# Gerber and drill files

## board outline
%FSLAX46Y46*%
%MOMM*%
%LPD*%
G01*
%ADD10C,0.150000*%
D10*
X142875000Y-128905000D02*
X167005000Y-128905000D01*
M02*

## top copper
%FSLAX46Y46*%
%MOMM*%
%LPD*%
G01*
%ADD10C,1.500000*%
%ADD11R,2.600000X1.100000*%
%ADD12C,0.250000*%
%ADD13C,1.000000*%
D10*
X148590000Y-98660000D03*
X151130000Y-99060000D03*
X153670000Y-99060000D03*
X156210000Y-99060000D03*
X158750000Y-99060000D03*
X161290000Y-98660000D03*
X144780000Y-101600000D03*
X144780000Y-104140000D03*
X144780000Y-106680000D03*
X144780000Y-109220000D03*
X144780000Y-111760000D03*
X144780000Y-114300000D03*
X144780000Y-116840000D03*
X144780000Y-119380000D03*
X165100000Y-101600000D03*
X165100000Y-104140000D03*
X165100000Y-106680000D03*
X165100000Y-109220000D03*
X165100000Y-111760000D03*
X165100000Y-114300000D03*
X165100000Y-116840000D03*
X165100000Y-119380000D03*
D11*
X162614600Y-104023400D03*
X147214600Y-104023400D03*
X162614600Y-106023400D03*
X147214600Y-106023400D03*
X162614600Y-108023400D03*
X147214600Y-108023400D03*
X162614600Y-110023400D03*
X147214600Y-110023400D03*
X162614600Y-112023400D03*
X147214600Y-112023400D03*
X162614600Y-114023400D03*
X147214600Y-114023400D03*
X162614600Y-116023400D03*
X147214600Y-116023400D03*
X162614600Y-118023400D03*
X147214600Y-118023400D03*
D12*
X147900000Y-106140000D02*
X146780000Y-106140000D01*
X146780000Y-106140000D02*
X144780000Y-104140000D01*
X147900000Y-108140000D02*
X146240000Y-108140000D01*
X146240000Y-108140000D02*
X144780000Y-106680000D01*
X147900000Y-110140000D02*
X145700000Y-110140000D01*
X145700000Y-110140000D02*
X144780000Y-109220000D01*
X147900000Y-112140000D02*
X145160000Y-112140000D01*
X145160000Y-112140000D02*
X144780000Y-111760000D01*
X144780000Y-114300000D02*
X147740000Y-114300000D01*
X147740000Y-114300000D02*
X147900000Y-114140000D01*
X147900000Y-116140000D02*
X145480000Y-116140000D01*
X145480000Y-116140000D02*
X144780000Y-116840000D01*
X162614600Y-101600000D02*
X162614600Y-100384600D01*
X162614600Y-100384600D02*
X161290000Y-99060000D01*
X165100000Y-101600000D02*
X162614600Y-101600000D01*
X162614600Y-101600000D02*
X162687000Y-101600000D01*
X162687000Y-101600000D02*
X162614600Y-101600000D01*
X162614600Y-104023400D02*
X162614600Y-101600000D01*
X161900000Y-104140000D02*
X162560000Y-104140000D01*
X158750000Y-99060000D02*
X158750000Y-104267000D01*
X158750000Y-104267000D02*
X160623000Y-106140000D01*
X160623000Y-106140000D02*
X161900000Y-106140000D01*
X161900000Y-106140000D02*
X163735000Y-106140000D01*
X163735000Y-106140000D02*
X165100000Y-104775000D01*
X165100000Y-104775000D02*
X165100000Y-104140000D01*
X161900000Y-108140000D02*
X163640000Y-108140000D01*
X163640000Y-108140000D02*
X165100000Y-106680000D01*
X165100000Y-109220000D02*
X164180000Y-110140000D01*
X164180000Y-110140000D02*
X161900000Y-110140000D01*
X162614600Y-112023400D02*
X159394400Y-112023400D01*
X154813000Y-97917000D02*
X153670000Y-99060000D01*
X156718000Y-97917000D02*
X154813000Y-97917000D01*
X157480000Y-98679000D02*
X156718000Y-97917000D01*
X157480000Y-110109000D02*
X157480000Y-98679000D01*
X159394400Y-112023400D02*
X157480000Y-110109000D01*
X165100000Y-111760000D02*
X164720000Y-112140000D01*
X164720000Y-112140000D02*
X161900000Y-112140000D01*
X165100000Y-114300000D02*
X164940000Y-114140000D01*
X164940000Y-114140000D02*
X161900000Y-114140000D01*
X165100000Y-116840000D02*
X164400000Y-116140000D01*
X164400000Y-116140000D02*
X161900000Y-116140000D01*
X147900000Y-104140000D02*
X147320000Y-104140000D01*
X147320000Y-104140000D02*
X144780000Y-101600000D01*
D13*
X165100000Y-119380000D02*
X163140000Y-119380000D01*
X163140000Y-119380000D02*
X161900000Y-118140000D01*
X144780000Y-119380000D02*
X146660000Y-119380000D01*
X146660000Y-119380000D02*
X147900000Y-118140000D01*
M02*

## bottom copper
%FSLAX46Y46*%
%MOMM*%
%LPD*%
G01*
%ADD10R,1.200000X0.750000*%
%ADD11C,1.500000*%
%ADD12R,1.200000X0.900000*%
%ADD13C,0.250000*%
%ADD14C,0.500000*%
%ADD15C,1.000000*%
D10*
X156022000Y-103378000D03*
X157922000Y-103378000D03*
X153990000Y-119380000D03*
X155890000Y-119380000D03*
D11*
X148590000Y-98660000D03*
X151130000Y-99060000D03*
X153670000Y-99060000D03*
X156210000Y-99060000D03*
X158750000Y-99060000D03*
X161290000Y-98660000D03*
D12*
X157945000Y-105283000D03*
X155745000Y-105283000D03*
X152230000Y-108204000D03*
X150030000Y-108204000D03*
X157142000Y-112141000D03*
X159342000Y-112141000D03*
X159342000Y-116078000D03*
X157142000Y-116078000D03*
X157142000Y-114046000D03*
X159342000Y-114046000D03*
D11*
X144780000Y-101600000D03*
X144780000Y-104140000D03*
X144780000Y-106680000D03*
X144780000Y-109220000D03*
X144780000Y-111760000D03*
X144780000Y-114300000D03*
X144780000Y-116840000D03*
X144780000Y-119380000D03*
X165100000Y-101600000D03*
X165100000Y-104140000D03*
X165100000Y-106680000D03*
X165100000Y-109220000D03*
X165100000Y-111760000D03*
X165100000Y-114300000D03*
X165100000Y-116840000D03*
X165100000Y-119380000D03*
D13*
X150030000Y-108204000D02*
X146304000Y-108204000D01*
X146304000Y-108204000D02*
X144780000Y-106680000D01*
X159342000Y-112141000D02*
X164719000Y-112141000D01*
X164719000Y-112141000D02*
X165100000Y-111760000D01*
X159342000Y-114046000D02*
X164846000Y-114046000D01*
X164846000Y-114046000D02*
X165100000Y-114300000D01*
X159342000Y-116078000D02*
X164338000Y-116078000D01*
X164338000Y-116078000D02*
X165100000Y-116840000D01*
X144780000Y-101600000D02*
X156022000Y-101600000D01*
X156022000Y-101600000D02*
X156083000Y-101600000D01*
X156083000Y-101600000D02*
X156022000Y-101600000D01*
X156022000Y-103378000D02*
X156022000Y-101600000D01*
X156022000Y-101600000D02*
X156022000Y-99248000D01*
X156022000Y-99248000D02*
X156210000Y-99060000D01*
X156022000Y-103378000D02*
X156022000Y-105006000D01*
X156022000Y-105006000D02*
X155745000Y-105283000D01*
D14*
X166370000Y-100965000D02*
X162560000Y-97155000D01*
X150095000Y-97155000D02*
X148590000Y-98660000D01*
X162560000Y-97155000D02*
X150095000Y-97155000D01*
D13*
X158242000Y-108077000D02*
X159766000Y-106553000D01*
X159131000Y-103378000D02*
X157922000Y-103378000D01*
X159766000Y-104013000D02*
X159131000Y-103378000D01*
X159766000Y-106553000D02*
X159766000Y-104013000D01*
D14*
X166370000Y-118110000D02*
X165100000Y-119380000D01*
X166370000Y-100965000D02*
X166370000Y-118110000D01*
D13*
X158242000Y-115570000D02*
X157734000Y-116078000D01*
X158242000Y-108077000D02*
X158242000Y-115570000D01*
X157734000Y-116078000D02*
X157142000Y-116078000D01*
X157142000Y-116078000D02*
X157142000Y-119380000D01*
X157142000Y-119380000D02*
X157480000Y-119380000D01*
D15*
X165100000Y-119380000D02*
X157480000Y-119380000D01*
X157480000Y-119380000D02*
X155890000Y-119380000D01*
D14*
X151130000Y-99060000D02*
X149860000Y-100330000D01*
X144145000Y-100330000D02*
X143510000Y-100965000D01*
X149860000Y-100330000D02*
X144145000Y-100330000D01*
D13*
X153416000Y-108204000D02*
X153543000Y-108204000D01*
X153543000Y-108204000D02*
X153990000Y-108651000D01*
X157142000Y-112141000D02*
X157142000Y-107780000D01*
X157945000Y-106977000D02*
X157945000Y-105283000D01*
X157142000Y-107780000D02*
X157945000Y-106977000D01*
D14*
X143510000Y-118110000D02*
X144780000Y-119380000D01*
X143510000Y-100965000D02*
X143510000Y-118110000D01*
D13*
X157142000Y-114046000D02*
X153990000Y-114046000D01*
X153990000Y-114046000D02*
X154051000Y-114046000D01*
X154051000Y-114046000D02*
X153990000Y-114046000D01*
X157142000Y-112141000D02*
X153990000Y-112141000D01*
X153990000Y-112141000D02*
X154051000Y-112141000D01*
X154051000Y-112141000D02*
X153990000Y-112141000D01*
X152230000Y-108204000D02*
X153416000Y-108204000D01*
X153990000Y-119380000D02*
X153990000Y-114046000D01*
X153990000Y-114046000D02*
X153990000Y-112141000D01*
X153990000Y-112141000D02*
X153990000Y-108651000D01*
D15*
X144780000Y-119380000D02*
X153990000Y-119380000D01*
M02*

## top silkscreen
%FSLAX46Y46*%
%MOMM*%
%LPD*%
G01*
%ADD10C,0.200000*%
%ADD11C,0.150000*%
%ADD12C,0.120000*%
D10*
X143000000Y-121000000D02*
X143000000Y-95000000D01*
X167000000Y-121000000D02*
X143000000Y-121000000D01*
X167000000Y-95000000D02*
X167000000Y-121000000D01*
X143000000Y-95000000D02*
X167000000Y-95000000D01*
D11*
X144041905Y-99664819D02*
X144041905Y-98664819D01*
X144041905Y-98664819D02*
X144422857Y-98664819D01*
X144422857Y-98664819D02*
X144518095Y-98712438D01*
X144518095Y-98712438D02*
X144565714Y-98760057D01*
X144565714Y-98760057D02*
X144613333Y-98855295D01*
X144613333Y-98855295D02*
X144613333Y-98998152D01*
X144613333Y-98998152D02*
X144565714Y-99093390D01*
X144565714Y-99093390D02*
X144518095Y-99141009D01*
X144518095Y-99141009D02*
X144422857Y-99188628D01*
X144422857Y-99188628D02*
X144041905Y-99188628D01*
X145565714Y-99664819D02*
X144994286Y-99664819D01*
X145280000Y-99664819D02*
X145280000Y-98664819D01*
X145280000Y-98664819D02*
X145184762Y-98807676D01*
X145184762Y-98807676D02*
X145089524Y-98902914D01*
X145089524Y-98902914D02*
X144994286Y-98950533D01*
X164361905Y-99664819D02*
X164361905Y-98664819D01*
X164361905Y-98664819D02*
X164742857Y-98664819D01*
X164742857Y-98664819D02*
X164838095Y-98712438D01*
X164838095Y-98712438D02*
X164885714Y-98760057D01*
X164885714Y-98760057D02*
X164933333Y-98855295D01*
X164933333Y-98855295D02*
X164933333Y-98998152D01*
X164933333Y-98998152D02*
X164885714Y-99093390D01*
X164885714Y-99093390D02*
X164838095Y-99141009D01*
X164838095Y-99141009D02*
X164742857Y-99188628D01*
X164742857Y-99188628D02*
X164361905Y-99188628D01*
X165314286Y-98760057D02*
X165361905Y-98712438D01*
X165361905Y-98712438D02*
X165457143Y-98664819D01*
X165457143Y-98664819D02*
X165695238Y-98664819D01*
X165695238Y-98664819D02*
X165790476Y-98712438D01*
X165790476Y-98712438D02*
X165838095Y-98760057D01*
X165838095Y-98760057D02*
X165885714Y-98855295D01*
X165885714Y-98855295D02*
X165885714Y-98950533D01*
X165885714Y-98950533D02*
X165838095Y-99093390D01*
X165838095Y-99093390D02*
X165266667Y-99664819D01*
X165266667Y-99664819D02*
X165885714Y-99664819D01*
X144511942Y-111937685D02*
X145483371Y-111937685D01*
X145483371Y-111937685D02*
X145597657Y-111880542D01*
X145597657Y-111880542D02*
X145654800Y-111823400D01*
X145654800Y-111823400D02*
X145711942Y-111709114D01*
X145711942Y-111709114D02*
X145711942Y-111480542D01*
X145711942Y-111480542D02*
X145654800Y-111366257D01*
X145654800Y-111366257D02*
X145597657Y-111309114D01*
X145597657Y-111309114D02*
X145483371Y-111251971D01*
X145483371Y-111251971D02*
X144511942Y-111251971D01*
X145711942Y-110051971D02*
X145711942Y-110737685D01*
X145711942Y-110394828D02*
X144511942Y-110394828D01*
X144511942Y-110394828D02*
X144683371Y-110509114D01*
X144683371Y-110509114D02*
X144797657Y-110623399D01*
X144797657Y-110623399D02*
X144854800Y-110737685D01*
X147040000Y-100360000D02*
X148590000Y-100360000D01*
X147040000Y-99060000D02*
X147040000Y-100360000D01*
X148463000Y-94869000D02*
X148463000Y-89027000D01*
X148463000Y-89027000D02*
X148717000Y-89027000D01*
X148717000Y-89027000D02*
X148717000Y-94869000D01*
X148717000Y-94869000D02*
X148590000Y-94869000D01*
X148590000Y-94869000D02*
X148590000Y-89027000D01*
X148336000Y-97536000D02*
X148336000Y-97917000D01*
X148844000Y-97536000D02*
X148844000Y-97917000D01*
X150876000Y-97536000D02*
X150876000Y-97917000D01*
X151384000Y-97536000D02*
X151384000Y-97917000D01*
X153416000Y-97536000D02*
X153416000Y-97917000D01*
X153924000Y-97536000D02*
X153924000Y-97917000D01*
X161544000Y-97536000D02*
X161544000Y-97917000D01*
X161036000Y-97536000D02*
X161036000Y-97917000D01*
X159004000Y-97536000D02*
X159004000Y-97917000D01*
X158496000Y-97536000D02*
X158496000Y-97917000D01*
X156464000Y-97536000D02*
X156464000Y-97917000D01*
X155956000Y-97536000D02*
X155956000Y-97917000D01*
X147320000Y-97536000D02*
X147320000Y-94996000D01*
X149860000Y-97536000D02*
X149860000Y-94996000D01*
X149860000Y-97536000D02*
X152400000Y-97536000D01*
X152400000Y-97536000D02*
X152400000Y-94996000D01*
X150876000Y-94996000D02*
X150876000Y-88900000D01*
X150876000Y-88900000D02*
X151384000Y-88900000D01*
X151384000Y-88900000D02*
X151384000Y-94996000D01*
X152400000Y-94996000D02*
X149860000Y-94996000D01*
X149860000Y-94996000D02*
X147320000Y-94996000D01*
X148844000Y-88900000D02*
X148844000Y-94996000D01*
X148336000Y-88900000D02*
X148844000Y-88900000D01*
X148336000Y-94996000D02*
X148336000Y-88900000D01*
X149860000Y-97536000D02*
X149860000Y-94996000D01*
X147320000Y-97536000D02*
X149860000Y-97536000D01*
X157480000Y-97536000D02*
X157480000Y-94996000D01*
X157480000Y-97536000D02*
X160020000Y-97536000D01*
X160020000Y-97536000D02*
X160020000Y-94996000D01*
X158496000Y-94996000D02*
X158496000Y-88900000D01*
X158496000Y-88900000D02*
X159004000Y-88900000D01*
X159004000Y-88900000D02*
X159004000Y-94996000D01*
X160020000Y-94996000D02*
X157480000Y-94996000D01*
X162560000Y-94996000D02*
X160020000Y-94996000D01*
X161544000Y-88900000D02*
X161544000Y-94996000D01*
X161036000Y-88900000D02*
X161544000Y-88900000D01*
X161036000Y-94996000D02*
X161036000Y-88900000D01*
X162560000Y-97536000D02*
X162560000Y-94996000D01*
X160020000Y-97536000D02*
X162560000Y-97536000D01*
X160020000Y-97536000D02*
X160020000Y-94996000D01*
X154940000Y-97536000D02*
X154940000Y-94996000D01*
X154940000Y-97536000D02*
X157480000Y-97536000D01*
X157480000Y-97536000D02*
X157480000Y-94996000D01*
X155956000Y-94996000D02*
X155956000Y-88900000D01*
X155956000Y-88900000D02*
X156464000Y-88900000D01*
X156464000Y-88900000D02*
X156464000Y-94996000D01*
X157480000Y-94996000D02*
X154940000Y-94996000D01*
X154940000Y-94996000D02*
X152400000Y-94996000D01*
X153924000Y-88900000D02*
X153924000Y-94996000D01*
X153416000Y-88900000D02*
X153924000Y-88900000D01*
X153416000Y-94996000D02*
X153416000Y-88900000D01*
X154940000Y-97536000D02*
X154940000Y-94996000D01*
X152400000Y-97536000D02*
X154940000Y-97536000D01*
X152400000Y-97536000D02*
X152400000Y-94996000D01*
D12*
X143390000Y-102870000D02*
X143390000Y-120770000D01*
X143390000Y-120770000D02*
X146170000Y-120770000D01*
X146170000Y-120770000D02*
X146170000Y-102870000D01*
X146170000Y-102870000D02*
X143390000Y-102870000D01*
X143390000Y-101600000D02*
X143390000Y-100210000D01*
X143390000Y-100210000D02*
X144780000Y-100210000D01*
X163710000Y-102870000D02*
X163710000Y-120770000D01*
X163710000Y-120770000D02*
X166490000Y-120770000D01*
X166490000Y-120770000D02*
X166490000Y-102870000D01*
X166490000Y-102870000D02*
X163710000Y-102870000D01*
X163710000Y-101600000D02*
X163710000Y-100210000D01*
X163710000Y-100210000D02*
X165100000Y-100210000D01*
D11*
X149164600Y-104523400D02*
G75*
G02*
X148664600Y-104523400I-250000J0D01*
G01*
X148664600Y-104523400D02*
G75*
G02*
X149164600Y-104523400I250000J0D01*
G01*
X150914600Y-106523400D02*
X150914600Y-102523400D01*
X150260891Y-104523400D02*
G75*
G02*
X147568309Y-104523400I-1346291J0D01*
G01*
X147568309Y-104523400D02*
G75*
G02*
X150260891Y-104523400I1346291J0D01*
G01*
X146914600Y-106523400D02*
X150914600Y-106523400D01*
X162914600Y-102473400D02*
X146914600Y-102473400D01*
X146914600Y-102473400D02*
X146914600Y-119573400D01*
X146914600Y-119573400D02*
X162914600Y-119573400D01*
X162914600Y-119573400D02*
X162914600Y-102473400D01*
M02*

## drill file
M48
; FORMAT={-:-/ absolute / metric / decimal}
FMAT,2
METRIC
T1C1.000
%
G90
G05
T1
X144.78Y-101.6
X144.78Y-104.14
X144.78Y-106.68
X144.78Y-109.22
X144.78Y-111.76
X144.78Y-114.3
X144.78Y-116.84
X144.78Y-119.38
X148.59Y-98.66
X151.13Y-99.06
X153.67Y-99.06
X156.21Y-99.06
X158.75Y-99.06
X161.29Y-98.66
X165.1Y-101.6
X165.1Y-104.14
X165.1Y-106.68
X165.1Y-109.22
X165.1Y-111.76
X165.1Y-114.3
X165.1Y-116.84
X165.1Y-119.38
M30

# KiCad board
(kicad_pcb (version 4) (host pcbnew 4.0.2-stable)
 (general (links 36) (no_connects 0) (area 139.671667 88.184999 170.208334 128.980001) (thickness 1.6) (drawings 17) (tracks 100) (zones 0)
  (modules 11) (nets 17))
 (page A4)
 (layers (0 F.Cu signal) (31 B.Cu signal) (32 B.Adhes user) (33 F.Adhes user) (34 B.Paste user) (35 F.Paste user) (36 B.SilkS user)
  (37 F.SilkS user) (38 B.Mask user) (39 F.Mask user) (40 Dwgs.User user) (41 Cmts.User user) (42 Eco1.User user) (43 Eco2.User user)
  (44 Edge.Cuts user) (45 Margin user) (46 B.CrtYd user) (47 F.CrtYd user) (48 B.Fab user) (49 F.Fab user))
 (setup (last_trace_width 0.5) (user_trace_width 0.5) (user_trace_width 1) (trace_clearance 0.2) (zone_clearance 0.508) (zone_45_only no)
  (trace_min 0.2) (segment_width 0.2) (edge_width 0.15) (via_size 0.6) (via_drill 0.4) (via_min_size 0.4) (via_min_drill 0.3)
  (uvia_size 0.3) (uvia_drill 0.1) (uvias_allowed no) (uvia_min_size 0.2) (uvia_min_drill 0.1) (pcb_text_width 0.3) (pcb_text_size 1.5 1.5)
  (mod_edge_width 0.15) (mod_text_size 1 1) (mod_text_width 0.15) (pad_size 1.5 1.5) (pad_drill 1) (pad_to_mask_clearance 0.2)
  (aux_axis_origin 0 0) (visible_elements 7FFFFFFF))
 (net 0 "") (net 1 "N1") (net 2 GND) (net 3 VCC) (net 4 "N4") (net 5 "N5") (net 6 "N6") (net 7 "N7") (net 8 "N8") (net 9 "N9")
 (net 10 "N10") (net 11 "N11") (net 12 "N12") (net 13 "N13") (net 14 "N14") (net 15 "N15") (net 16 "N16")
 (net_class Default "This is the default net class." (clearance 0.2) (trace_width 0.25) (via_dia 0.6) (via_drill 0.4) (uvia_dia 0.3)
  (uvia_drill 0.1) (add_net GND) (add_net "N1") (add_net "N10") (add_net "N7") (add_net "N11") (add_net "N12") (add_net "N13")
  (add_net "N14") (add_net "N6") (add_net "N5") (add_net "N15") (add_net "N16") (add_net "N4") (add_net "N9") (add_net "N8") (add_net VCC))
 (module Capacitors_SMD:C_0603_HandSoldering (layer B.Cu) (at 156.972 103.378)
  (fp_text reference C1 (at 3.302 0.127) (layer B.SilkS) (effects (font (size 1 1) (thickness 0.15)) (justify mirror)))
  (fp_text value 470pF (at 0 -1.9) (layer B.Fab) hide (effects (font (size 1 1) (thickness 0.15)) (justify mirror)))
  (pad 1 smd rect (at -0.95 0) (size 1.2 0.75) (layers B.Cu B.Paste B.Mask) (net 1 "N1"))
  (pad 2 smd rect (at 0.95 0) (size 1.2 0.75) (layers B.Cu B.Paste B.Mask) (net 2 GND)))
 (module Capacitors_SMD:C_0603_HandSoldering (layer B.Cu) (at 154.94 119.38)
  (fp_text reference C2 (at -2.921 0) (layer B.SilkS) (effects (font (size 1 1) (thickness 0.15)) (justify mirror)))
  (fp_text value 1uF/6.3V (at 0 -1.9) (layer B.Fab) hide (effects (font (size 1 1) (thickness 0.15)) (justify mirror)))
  (pad 1 smd rect (at -0.95 0) (size 1.2 0.75) (layers B.Cu B.Paste B.Mask) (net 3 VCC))
  (pad 2 smd rect (at 0.95 0) (size 1.2 0.75) (layers B.Cu B.Paste B.Mask) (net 2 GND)))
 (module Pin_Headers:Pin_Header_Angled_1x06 (layer F.Cu) (at 148.59 99.06 90)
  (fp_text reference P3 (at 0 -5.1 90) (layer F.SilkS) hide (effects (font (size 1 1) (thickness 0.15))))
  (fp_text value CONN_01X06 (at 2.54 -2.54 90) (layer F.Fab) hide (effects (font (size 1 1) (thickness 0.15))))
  (fp_line (start -1.3 -1.55) (end -1.3 0) (layer F.SilkS) (width 0.15))
  (fp_line (start 0 -1.55) (end -1.3 -1.55) (layer F.SilkS) (width 0.15))
  (fp_line (start 4.191 -0.127) (end 10.033 -0.127) (layer F.SilkS) (width 0.15))
  (fp_line (start 10.033 -0.127) (end 10.033 0.127) (layer F.SilkS) (width 0.15))
  (fp_line (start 10.033 0.127) (end 4.191 0.127) (layer F.SilkS) (width 0.15))
  (fp_line (start 4.191 0.127) (end 4.191 0) (layer F.SilkS) (width 0.15))
  (fp_line (start 4.191 0) (end 10.033 0) (layer F.SilkS) (width 0.15))
  (fp_line (start 1.524 -0.254) (end 1.143 -0.254) (layer F.SilkS) (width 0.15))
  (fp_line (start 1.524 0.254) (end 1.143 0.254) (layer F.SilkS) (width 0.15))
  (fp_line (start 1.524 2.286) (end 1.143 2.286) (layer F.SilkS) (width 0.15))
  (fp_line (start 1.524 2.794) (end 1.143 2.794) (layer F.SilkS) (width 0.15))
  (fp_line (start 1.524 4.826) (end 1.143 4.826) (layer F.SilkS) (width 0.15))
  (fp_line (start 1.524 5.334) (end 1.143 5.334) (layer F.SilkS) (width 0.15))
  (fp_line (start 1.524 12.954) (end 1.143 12.954) (layer F.SilkS) (width 0.15))
  (fp_line (start 1.524 12.446) (end 1.143 12.446) (layer F.SilkS) (width 0.15))
  (fp_line (start 1.524 10.414) (end 1.143 10.414) (layer F.SilkS) (width 0.15))
  (fp_line (start 1.524 9.906) (end 1.143 9.906) (layer F.SilkS) (width 0.15))
  (fp_line (start 1.524 7.874) (end 1.143 7.874) (layer F.SilkS) (width 0.15))
  (fp_line (start 1.524 7.366) (end 1.143 7.366) (layer F.SilkS) (width 0.15))
  (fp_line (start 1.524 -1.27) (end 4.064 -1.27) (layer F.SilkS) (width 0.15))
  (fp_line (start 1.524 1.27) (end 4.064 1.27) (layer F.SilkS) (width 0.15))
  (fp_line (start 1.524 1.27) (end 1.524 3.81) (layer F.SilkS) (width 0.15))
  (fp_line (start 1.524 3.81) (end 4.064 3.81) (layer F.SilkS) (width 0.15))
  (fp_line (start 4.064 2.286) (end 10.16 2.286) (layer F.SilkS) (width 0.15))
  (fp_line (start 10.16 2.286) (end 10.16 2.794) (layer F.SilkS) (width 0.15))
  (fp_line (start 10.16 2.794) (end 4.064 2.794) (layer F.SilkS) (width 0.15))
  (fp_line (start 4.064 3.81) (end 4.064 1.27) (layer F.SilkS) (width 0.15))
  (fp_line (start 4.064 1.27) (end 4.064 -1.27) (layer F.SilkS) (width 0.15))
  (fp_line (start 10.16 0.254) (end 4.064 0.254) (layer F.SilkS) (width 0.15))
  (fp_line (start 10.16 -0.254) (end 10.16 0.254) (layer F.SilkS) (width 0.15))
  (fp_line (start 4.064 -0.254) (end 10.16 -0.254) (layer F.SilkS) (width 0.15))
  (fp_line (start 1.524 1.27) (end 4.064 1.27) (layer F.SilkS) (width 0.15))
  (fp_line (start 1.524 -1.27) (end 1.524 1.27) (layer F.SilkS) (width 0.15))
  (fp_line (start 1.524 8.89) (end 4.064 8.89) (layer F.SilkS) (width 0.15))
  (fp_line (start 1.524 8.89) (end 1.524 11.43) (layer F.SilkS) (width 0.15))
  (fp_line (start 1.524 11.43) (end 4.064 11.43) (layer F.SilkS) (width 0.15))
  (fp_line (start 4.064 9.906) (end 10.16 9.906) (layer F.SilkS) (width 0.15))
  (fp_line (start 10.16 9.906) (end 10.16 10.414) (layer F.SilkS) (width 0.15))
  (fp_line (start 10.16 10.414) (end 4.064 10.414) (layer F.SilkS) (width 0.15))
  (fp_line (start 4.064 11.43) (end 4.064 8.89) (layer F.SilkS) (width 0.15))
  (fp_line (start 4.064 13.97) (end 4.064 11.43) (layer F.SilkS) (width 0.15))
  (fp_line (start 10.16 12.954) (end 4.064 12.954) (layer F.SilkS) (width 0.15))
  (fp_line (start 10.16 12.446) (end 10.16 12.954) (layer F.SilkS) (width 0.15))
  (fp_line (start 4.064 12.446) (end 10.16 12.446) (layer F.SilkS) (width 0.15))
  (fp_line (start 1.524 13.97) (end 4.064 13.97) (layer F.SilkS) (width 0.15))
  (fp_line (start 1.524 11.43) (end 1.524 13.97) (layer F.SilkS) (width 0.15))
  (fp_line (start 1.524 11.43) (end 4.064 11.43) (layer F.SilkS) (width 0.15))
  (fp_line (start 1.524 6.35) (end 4.064 6.35) (layer F.SilkS) (width 0.15))
  (fp_line (start 1.524 6.35) (end 1.524 8.89) (layer F.SilkS) (width 0.15))
  (fp_line (start 1.524 8.89) (end 4.064 8.89) (layer F.SilkS) (width 0.15))
  (fp_line (start 4.064 7.366) (end 10.16 7.366) (layer F.SilkS) (width 0.15))
  (fp_line (start 10.16 7.366) (end 10.16 7.874) (layer F.SilkS) (width 0.15))
  (fp_line (start 10.16 7.874) (end 4.064 7.874) (layer F.SilkS) (width 0.15))
  (fp_line (start 4.064 8.89) (end 4.064 6.35) (layer F.SilkS) (width 0.15))
  (fp_line (start 4.064 6.35) (end 4.064 3.81) (layer F.SilkS) (width 0.15))
  (fp_line (start 10.16 5.334) (end 4.064 5.334) (layer F.SilkS) (width 0.15))
  (fp_line (start 10.16 4.826) (end 10.16 5.334) (layer F.SilkS) (width 0.15))
  (fp_line (start 4.064 4.826) (end 10.16 4.826) (layer F.SilkS) (width 0.15))
  (fp_line (start 1.524 6.35) (end 4.064 6.35) (layer F.SilkS) (width 0.15))
  (fp_line (start 1.524 3.81) (end 1.524 6.35) (layer F.SilkS) (width 0.15))
  (fp_line (start 1.524 3.81) (end 4.064 3.81) (layer F.SilkS) (width 0.15))
  (pad 1 thru_hole circle (at 0.4 0 90) (size 1.5 1.5) (drill 1) (layers *.Cu *.Mask) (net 2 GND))
  (pad 2 thru_hole circle (at 0 2.54 90) (size 1.5 1.5) (drill 1) (layers *.Cu *.Mask) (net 3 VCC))
  (pad 3 thru_hole circle (at 0 5.08 90) (size 1.5 1.5) (drill 1) (layers *.Cu *.Mask) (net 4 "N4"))
  (pad 4 thru_hole circle (at 0 7.62 90) (size 1.5 1.5) (drill 1) (layers *.Cu *.Mask) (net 1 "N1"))
  (pad 5 thru_hole circle (at 0 10.16 90) (size 1.5 1.5) (drill 1) (layers *.Cu *.Mask) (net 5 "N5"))
  (pad 6 thru_hole circle (at 0.4 12.7 90) (size 1.5 1.5) (drill 1) (layers *.Cu *.Mask) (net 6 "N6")))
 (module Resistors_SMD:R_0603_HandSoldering (layer B.Cu) (at 156.845 105.283 180)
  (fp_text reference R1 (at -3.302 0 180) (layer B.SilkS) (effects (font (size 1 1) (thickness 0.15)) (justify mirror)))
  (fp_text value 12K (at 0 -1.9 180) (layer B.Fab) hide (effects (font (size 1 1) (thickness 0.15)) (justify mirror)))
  (pad 1 smd rect (at -1.1 0 180) (size 1.2 0.9) (layers B.Cu B.Paste B.Mask) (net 3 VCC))
  (pad 2 smd rect (at 1.1 0 180) (size 1.2 0.9) (layers B.Cu B.Paste B.Mask) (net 1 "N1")))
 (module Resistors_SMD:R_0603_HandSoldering (layer B.Cu) (at 151.13 108.204 180)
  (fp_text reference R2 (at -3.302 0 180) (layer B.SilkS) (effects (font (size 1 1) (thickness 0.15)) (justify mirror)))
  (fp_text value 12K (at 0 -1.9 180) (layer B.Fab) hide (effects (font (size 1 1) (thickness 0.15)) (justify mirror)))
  (pad 1 smd rect (at -1.1 0 180) (size 1.2 0.9) (layers B.Cu B.Paste B.Mask) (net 3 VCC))
  (pad 2 smd rect (at 1.1 0 180) (size 1.2 0.9) (layers B.Cu B.Paste B.Mask) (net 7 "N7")))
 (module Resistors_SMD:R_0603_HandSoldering (layer B.Cu) (at 158.242 112.141)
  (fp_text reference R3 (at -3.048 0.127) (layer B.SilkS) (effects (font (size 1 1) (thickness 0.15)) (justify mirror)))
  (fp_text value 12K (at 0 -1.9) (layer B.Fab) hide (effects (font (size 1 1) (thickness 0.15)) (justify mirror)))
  (pad 1 smd rect (at -1.1 0) (size 1.2 0.9) (layers B.Cu B.Paste B.Mask) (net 3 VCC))
  (pad 2 smd rect (at 1.1 0) (size 1.2 0.9) (layers B.Cu B.Paste B.Mask) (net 4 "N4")))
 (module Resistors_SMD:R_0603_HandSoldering (layer B.Cu) (at 158.242 116.078 180)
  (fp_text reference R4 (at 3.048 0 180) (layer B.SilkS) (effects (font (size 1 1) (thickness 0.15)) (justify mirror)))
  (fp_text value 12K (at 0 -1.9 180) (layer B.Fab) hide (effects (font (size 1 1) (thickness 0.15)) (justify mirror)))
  (pad 1 smd rect (at -1.1 0 180) (size 1.2 0.9) (layers B.Cu B.Paste B.Mask) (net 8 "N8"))
  (pad 2 smd rect (at 1.1 0 180) (size 1.2 0.9) (layers B.Cu B.Paste B.Mask) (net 2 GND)))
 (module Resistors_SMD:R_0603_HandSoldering (layer B.Cu) (at 158.242 114.046)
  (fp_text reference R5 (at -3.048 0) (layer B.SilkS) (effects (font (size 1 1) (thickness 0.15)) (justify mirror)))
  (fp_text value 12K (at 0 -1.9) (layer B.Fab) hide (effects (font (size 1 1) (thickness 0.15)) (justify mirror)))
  (pad 1 smd rect (at -1.1 0) (size 1.2 0.9) (layers B.Cu B.Paste B.Mask) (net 3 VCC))
  (pad 2 smd rect (at 1.1 0) (size 1.2 0.9) (layers B.Cu B.Paste B.Mask) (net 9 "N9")))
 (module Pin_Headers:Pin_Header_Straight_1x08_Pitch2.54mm (layer F.Cu) (at 144.78 101.6)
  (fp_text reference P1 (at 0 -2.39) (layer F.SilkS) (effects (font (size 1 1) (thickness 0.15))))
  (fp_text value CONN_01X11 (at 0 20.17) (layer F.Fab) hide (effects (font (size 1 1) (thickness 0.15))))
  (fp_line (start -1.39 1.27) (end -1.39 19.17) (layer F.SilkS) (width 0.12))
  (fp_line (start -1.39 19.17) (end 1.39 19.17) (layer F.SilkS) (width 0.12))
  (fp_line (start 1.39 19.17) (end 1.39 1.27) (layer F.SilkS) (width 0.12))
  (fp_line (start 1.39 1.27) (end -1.39 1.27) (layer F.SilkS) (width 0.12))
  (fp_line (start -1.39 0) (end -1.39 -1.39) (layer F.SilkS) (width 0.12))
  (fp_line (start -1.39 -1.39) (end 0 -1.39) (layer F.SilkS) (width 0.12))
  (pad 1 thru_hole circle (at 0 0) (size 1.5 1.5) (drill 1) (layers *.Cu *.Mask) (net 1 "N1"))
  (pad 2 thru_hole circle (at 0 2.54) (size 1.5 1.5) (drill 1) (layers *.Cu *.Mask) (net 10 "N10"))
  (pad 3 thru_hole circle (at 0 5.08) (size 1.5 1.5) (drill 1) (layers *.Cu *.Mask) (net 7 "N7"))
  (pad 4 thru_hole circle (at 0 7.62) (size 1.5 1.5) (drill 1) (layers *.Cu *.Mask) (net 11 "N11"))
  (pad 5 thru_hole circle (at 0 10.16) (size 1.5 1.5) (drill 1) (layers *.Cu *.Mask) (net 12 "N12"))
  (pad 6 thru_hole circle (at 0 12.7) (size 1.5 1.5) (drill 1) (layers *.Cu *.Mask) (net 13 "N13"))
  (pad 7 thru_hole circle (at 0 15.24) (size 1.5 1.5) (drill 1) (layers *.Cu *.Mask) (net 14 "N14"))
  (pad 8 thru_hole circle (at 0 17.78) (size 1.5 1.5) (drill 1) (layers *.Cu *.Mask) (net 3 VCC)))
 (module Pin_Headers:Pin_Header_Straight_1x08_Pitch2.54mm (layer F.Cu) (at 165.1 101.6)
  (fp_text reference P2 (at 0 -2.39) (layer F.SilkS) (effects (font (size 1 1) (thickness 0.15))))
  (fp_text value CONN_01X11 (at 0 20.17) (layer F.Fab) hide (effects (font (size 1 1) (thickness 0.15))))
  (fp_line (start -1.39 1.27) (end -1.39 19.17) (layer F.SilkS) (width 0.12))
  (fp_line (start -1.39 19.17) (end 1.39 19.17) (layer F.SilkS) (width 0.12))
  (fp_line (start 1.39 19.17) (end 1.39 1.27) (layer F.SilkS) (width 0.12))
  (fp_line (start 1.39 1.27) (end -1.39 1.27) (layer F.SilkS) (width 0.12))
  (fp_line (start -1.39 0) (end -1.39 -1.39) (layer F.SilkS) (width 0.12))
  (fp_line (start -1.39 -1.39) (end 0 -1.39) (layer F.SilkS) (width 0.12))
  (pad 1 thru_hole circle (at 0 0) (size 1.5 1.5) (drill 1) (layers *.Cu *.Mask) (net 6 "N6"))
  (pad 2 thru_hole circle (at 0 2.54) (size 1.5 1.5) (drill 1) (layers *.Cu *.Mask) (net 5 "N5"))
  (pad 3 thru_hole circle (at 0 5.08) (size 1.5 1.5) (drill 1) (layers *.Cu *.Mask) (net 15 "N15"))
  (pad 4 thru_hole circle (at 0 7.62) (size 1.5 1.5) (drill 1) (layers *.Cu *.Mask) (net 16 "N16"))
  (pad 5 thru_hole circle (at 0 10.16) (size 1.5 1.5) (drill 1) (layers *.Cu *.Mask) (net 4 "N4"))
  (pad 6 thru_hole circle (at 0 12.7) (size 1.5 1.5) (drill 1) (layers *.Cu *.Mask) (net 9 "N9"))
  (pad 7 thru_hole circle (at 0 15.24) (size 1.5 1.5) (drill 1) (layers *.Cu *.Mask) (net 8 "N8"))
  (pad 8 thru_hole circle (at 0 17.78) (size 1.5 1.5) (drill 1) (layers *.Cu *.Mask) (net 2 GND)))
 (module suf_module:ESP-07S (layer F.Cu) (at 154.9146 111.0234)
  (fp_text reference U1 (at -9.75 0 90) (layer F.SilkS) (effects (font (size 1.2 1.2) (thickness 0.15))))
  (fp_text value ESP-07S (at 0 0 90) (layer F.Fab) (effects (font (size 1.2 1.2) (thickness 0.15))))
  (fp_circle (center -6 -6.5) (end -6 -6.75) (layer F.SilkS) (width 0.15))
  (fp_line (start -4 -4.5) (end -4 -8.5) (layer F.SilkS) (width 0.15))
  (fp_circle (center -6 -6.5) (end -5.5 -7.75) (layer F.SilkS) (width 0.15))
  (fp_line (start -8 -4.5) (end -4 -4.5) (layer F.SilkS) (width 0.15))
  (fp_line (start 8 -8.55) (end -8 -8.55) (layer F.SilkS) (width 0.15))
  (fp_line (start -8 -8.55) (end -8 8.55) (layer F.SilkS) (width 0.15))
  (fp_line (start -8 8.55) (end 8 8.55) (layer F.SilkS) (width 0.15))
  (fp_line (start 8 8.55) (end 8 -8.55) (layer F.SilkS) (width 0.15))
  (pad 16 smd rect (at 7.7 -7 270) (size 1.1 2.6) (layers F.Cu F.Paste F.Mask) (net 6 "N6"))
  (pad 1 smd rect (at -7.7 -7 270) (size 1.1 2.6) (layers F.Cu F.Paste F.Mask) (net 1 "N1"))
  (pad 15 smd rect (at 7.7 -5 270) (size 1.1 2.6) (layers F.Cu F.Paste F.Mask) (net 5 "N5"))
  (pad 2 smd rect (at -7.7 -5 270) (size 1.1 2.6) (layers F.Cu F.Paste F.Mask) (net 10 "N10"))
  (pad 14 smd rect (at 7.7 -3 270) (size 1.1 2.6) (layers F.Cu F.Paste F.Mask) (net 15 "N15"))
  (pad 3 smd rect (at -7.7 -3 270) (size 1.1 2.6) (layers F.Cu F.Paste F.Mask) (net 7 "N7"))
  (pad 13 smd rect (at 7.7 -1 270) (size 1.1 2.6) (layers F.Cu F.Paste F.Mask) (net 16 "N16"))
  (pad 4 smd rect (at -7.7 -1 270) (size 1.1 2.6) (layers F.Cu F.Paste F.Mask) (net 11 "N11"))
  (pad 12 smd rect (at 7.7 1 270) (size 1.1 2.6) (layers F.Cu F.Paste F.Mask) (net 4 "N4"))
  (pad 5 smd rect (at -7.7 1 270) (size 1.1 2.6) (layers F.Cu F.Paste F.Mask) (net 12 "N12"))
  (pad 11 smd rect (at 7.7 3 270) (size 1.1 2.6) (layers F.Cu F.Paste F.Mask) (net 9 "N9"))
  (pad 6 smd rect (at -7.7 3 270) (size 1.1 2.6) (layers F.Cu F.Paste F.Mask) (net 13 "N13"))
  (pad 10 smd rect (at 7.7 5 270) (size 1.1 2.6) (layers F.Cu F.Paste F.Mask) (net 8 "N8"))
  (pad 7 smd rect (at -7.7 5 270) (size 1.1 2.6) (layers F.Cu F.Paste F.Mask) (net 14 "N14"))
  (pad 9 smd rect (at 7.7 7 270) (size 1.1 2.6) (layers F.Cu F.Paste F.Mask) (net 2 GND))
  (pad 8 smd rect (at -7.7 7 270) (size 1.1 2.6) (layers F.Cu F.Paste F.Mask) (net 3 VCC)))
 (gr_line (start 143 121) (end 143 95) (angle 90) (layer F.SilkS) (width 0.2))
 (gr_line (start 167 121) (end 143 121) (angle 90) (layer F.SilkS) (width 0.2))
 (gr_line (start 167 95) (end 167 121) (angle 90) (layer F.SilkS) (width 0.2))
 (gr_line (start 143 95) (end 167 95) (angle 90) (layer F.SilkS) (width 0.2))
 (gr_line (start 142.875 128.905) (end 167.005 128.905) (angle 90) (layer Edge.Cuts) (width 0.15))
 (segment (start 147.9 106.14) (end 146.78 106.14) (width 0.25) (layer F.Cu) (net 10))
 (segment (start 146.78 106.14) (end 144.78 104.14) (width 0.25) (layer F.Cu) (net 10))
 (segment (start 150.03 108.204) (end 146.304 108.204) (width 0.25) (layer B.Cu) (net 7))
 (segment (start 146.304 108.204) (end 144.78 106.68) (width 0.25) (layer B.Cu) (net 7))
 (segment (start 147.9 108.14) (end 146.24 108.14) (width 0.25) (layer F.Cu) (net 7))
 (segment (start 146.24 108.14) (end 144.78 106.68) (width 0.25) (layer F.Cu) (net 7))
 (segment (start 147.9 110.14) (end 145.7 110.14) (width 0.25) (layer F.Cu) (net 11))
 (segment (start 145.7 110.14) (end 144.78 109.22) (width 0.25) (layer F.Cu) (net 11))
 (segment (start 147.9 112.14) (end 145.16 112.14) (width 0.25) (layer F.Cu) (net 12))
 (segment (start 145.16 112.14) (end 144.78 111.76) (width 0.25) (layer F.Cu) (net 12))
 (segment (start 144.78 114.3) (end 147.74 114.3) (width 0.25) (layer F.Cu) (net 13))
 (segment (start 147.74 114.3) (end 147.9 114.14) (width 0.25) (layer F.Cu) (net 13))
 (segment (start 147.9 116.14) (end 145.48 116.14) (width 0.25) (layer F.Cu) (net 14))
 (segment (start 145.48 116.14) (end 144.78 116.84) (width 0.25) (layer F.Cu) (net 14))
 (segment (start 162.6146 101.6) (end 162.6146 100.3846) (width 0.25) (layer F.Cu) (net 6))
 (segment (start 162.6146 100.3846) (end 161.29 99.06) (width 0.25) (layer F.Cu) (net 6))
 (segment (start 165.1 101.6) (end 162.6146 101.6) (width 0.25) (layer F.Cu) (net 6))
 (segment (start 162.6146 101.6) (end 162.687 101.6) (width 0.25) (layer F.Cu) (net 6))
 (segment (start 162.687 101.6) (end 162.6146 101.6) (width 0.25) (layer F.Cu) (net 6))
 (segment (start 162.6146 104.0234) (end 162.6146 101.6) (width 0.25) (layer F.Cu) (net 6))
 (segment (start 161.9 104.14) (end 162.56 104.14) (width 0.25) (layer F.Cu) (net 6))
 (segment (start 158.75 99.06) (end 158.75 104.267) (width 0.25) (layer F.Cu) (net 5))
 (segment (start 158.75 104.267) (end 160.623 106.14) (width 0.25) (layer F.Cu) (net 5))
 (segment (start 160.623 106.14) (end 161.9 106.14) (width 0.25) (layer F.Cu) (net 5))
 (segment (start 161.9 106.14) (end 163.735 106.14) (width 0.25) (layer F.Cu) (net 5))
 (segment (start 163.735 106.14) (end 165.1 104.775) (width 0.25) (layer F.Cu) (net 5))
 (segment (start 165.1 104.775) (end 165.1 104.14) (width 0.25) (layer F.Cu) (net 5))
 (segment (start 161.9 108.14) (end 163.64 108.14) (width 0.25) (layer F.Cu) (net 15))
 (segment (start 163.64 108.14) (end 165.1 106.68) (width 0.25) (layer F.Cu) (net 15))
 (segment (start 165.1 109.22) (end 164.18 110.14) (width 0.25) (layer F.Cu) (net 16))
 (segment (start 164.18 110.14) (end 161.9 110.14) (width 0.25) (layer F.Cu) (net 16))
 (segment (start 162.6146 112.0234) (end 159.3944 112.0234) (width 0.25) (layer F.Cu) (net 4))
 (segment (start 154.813 97.917) (end 153.67 99.06) (width 0.25) (layer F.Cu) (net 4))
 (segment (start 156.718 97.917) (end 154.813 97.917) (width 0.25) (layer F.Cu) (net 4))
 (segment (start 157.48 98.679) (end 156.718 97.917) (width 0.25) (layer F.Cu) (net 4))
 (segment (start 157.48 110.109) (end 157.48 98.679) (width 0.25) (layer F.Cu) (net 4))
 (segment (start 159.3944 112.0234) (end 157.48 110.109) (width 0.25) (layer F.Cu) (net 4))
 (segment (start 159.342 112.141) (end 164.719 112.141) (width 0.25) (layer B.Cu) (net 4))
 (segment (start 164.719 112.141) (end 165.1 111.76) (width 0.25) (layer B.Cu) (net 4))
 (segment (start 165.1 111.76) (end 164.72 112.14) (width 0.25) (layer F.Cu) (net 4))
 (segment (start 164.72 112.14) (end 161.9 112.14) (width 0.25) (layer F.Cu) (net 4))
 (segment (start 159.342 114.046) (end 164.846 114.046) (width 0.25) (layer B.Cu) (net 9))
 (segment (start 164.846 114.046) (end 165.1 114.3) (width 0.25) (layer B.Cu) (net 9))
 (segment (start 165.1 114.3) (end 164.94 114.14) (width 0.25) (layer F.Cu) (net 9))
 (segment (start 164.94 114.14) (end 161.9 114.14) (width 0.25) (layer F.Cu) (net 9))
 (segment (start 159.342 116.078) (end 164.338 116.078) (width 0.25) (layer B.Cu) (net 8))
 (segment (start 164.338 116.078) (end 165.1 116.84) (width 0.25) (layer B.Cu) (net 8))
 (segment (start 165.1 116.84) (end 164.4 116.14) (width 0.25) (layer F.Cu) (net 8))
 (segment (start 164.4 116.14) (end 161.9 116.14) (width 0.25) (layer F.Cu) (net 8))
 (segment (start 144.78 101.6) (end 156.022 101.6) (width 0.25) (layer B.Cu) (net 1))
 (segment (start 156.022 101.6) (end 156.083 101.6) (width 0.25) (layer B.Cu) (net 1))
 (segment (start 156.083 101.6) (end 156.022 101.6) (width 0.25) (layer B.Cu) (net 1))
 (segment (start 156.022 103.378) (end 156.022 101.6) (width 0.25) (layer B.Cu) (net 1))
 (segment (start 156.022 101.6) (end 156.022 99.248) (width 0.25) (layer B.Cu) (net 1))
 (segment (start 156.022 99.248) (end 156.21 99.06) (width 0.25) (layer B.Cu) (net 1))
 (segment (start 156.022 103.378) (end 156.022 105.006) (width 0.25) (layer B.Cu) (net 1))
 (segment (start 156.022 105.006) (end 155.745 105.283) (width 0.25) (layer B.Cu) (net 1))
 (segment (start 147.9 104.14) (end 147.32 104.14) (width 0.25) (layer F.Cu) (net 1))
 (segment (start 147.32 104.14) (end 144.78 101.6) (width 0.25) (layer F.Cu) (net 1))
 (segment (start 166.37 100.965) (end 162.56 97.155) (width 0.5) (layer B.Cu) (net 2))
 (segment (start 150.095 97.155) (end 148.59 98.66) (width 0.5) (layer B.Cu) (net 2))
 (segment (start 162.56 97.155) (end 150.095 97.155) (width 0.5) (layer B.Cu) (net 2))
 (segment (start 158.242 108.077) (end 159.766 106.553) (width 0.25) (layer B.Cu) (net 2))
 (segment (start 159.131 103.378) (end 157.922 103.378) (width 0.25) (layer B.Cu) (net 2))
 (segment (start 159.766 104.013) (end 159.131 103.378) (width 0.25) (layer B.Cu) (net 2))
 (segment (start 159.766 106.553) (end 159.766 104.013) (width 0.25) (layer B.Cu) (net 2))
 (segment (start 166.37 118.11) (end 165.1 119.38) (width 0.5) (layer B.Cu) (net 2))
 (segment (start 166.37 100.965) (end 166.37 118.11) (width 0.5) (layer B.Cu) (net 2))
 (segment (start 158.242 115.57) (end 157.734 116.078) (width 0.25) (layer B.Cu) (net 2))
 (segment (start 158.242 108.077) (end 158.242 115.57) (width 0.25) (layer B.Cu) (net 2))
 (segment (start 157.734 116.078) (end 157.142 116.078) (width 0.25) (layer B.Cu) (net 2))
 (segment (start 157.142 116.078) (end 157.142 119.38) (width 0.25) (layer B.Cu) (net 2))
 (segment (start 157.142 119.38) (end 157.48 119.38) (width 0.25) (layer B.Cu) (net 2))
 (segment (start 165.1 119.38) (end 157.48 119.38) (width 1) (layer B.Cu) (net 2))
 (segment (start 157.48 119.38) (end 155.89 119.38) (width 1) (layer B.Cu) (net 2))
 (segment (start 165.1 119.38) (end 163.14 119.38) (width 1) (layer F.Cu) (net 2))
 (segment (start 163.14 119.38) (end 161.9 118.14) (width 1) (layer F.Cu) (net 2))
 (segment (start 151.13 99.06) (end 149.86 100.33) (width 0.5) (layer B.Cu) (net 3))
 (segment (start 144.145 100.33) (end 143.51 100.965) (width 0.5) (layer B.Cu) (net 3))
 (segment (start 149.86 100.33) (end 144.145 100.33) (width 0.5) (layer B.Cu) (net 3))
 (segment (start 153.416 108.204) (end 153.543 108.204) (width 0.25) (layer B.Cu) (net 3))
 (segment (start 153.543 108.204) (end 153.99 108.651) (width 0.25) (layer B.Cu) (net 3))
 (segment (start 157.142 112.141) (end 157.142 107.78) (width 0.25) (layer B.Cu) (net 3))
 (segment (start 157.945 106.977) (end 157.945 105.283) (width 0.25) (layer B.Cu) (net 3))
 (segment (start 157.142 107.78) (end 157.945 106.977) (width 0.25) (layer B.Cu) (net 3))
 (segment (start 143.51 118.11) (end 144.78 119.38) (width 0.5) (layer B.Cu) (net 3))
 (segment (start 143.51 100.965) (end 143.51 118.11) (width 0.5) (layer B.Cu) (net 3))
 (segment (start 157.142 114.046) (end 153.99 114.046) (width 0.25) (layer B.Cu) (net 3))
 (segment (start 153.99 114.046) (end 154.051 114.046) (width 0.25) (layer B.Cu) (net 3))
 (segment (start 154.051 114.046) (end 153.99 114.046) (width 0.25) (layer B.Cu) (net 3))
 (segment (start 157.142 112.141) (end 153.99 112.141) (width 0.25) (layer B.Cu) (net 3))
 (segment (start 153.99 112.141) (end 154.051 112.141) (width 0.25) (layer B.Cu) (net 3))
 (segment (start 154.051 112.141) (end 153.99 112.141) (width 0.25) (layer B.Cu) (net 3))
 (segment (start 152.23 108.204) (end 153.416 108.204) (width 0.25) (layer B.Cu) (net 3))
 (segment (start 153.99 119.38) (end 153.99 114.046) (width 0.25) (layer B.Cu) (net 3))
 (segment (start 153.99 114.046) (end 153.99 112.141) (width 0.25) (layer B.Cu) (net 3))
 (segment (start 153.99 112.141) (end 153.99 108.651) (width 0.25) (layer B.Cu) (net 3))
 (segment (start 144.78 119.38) (end 153.99 119.38) (width 1) (layer B.Cu) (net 3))
 (segment (start 144.78 119.38) (end 146.66 119.38) (width 1) (layer F.Cu) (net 3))
 (segment (start 146.66 119.38) (end 147.9 118.14) (width 1) (layer F.Cu) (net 3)))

